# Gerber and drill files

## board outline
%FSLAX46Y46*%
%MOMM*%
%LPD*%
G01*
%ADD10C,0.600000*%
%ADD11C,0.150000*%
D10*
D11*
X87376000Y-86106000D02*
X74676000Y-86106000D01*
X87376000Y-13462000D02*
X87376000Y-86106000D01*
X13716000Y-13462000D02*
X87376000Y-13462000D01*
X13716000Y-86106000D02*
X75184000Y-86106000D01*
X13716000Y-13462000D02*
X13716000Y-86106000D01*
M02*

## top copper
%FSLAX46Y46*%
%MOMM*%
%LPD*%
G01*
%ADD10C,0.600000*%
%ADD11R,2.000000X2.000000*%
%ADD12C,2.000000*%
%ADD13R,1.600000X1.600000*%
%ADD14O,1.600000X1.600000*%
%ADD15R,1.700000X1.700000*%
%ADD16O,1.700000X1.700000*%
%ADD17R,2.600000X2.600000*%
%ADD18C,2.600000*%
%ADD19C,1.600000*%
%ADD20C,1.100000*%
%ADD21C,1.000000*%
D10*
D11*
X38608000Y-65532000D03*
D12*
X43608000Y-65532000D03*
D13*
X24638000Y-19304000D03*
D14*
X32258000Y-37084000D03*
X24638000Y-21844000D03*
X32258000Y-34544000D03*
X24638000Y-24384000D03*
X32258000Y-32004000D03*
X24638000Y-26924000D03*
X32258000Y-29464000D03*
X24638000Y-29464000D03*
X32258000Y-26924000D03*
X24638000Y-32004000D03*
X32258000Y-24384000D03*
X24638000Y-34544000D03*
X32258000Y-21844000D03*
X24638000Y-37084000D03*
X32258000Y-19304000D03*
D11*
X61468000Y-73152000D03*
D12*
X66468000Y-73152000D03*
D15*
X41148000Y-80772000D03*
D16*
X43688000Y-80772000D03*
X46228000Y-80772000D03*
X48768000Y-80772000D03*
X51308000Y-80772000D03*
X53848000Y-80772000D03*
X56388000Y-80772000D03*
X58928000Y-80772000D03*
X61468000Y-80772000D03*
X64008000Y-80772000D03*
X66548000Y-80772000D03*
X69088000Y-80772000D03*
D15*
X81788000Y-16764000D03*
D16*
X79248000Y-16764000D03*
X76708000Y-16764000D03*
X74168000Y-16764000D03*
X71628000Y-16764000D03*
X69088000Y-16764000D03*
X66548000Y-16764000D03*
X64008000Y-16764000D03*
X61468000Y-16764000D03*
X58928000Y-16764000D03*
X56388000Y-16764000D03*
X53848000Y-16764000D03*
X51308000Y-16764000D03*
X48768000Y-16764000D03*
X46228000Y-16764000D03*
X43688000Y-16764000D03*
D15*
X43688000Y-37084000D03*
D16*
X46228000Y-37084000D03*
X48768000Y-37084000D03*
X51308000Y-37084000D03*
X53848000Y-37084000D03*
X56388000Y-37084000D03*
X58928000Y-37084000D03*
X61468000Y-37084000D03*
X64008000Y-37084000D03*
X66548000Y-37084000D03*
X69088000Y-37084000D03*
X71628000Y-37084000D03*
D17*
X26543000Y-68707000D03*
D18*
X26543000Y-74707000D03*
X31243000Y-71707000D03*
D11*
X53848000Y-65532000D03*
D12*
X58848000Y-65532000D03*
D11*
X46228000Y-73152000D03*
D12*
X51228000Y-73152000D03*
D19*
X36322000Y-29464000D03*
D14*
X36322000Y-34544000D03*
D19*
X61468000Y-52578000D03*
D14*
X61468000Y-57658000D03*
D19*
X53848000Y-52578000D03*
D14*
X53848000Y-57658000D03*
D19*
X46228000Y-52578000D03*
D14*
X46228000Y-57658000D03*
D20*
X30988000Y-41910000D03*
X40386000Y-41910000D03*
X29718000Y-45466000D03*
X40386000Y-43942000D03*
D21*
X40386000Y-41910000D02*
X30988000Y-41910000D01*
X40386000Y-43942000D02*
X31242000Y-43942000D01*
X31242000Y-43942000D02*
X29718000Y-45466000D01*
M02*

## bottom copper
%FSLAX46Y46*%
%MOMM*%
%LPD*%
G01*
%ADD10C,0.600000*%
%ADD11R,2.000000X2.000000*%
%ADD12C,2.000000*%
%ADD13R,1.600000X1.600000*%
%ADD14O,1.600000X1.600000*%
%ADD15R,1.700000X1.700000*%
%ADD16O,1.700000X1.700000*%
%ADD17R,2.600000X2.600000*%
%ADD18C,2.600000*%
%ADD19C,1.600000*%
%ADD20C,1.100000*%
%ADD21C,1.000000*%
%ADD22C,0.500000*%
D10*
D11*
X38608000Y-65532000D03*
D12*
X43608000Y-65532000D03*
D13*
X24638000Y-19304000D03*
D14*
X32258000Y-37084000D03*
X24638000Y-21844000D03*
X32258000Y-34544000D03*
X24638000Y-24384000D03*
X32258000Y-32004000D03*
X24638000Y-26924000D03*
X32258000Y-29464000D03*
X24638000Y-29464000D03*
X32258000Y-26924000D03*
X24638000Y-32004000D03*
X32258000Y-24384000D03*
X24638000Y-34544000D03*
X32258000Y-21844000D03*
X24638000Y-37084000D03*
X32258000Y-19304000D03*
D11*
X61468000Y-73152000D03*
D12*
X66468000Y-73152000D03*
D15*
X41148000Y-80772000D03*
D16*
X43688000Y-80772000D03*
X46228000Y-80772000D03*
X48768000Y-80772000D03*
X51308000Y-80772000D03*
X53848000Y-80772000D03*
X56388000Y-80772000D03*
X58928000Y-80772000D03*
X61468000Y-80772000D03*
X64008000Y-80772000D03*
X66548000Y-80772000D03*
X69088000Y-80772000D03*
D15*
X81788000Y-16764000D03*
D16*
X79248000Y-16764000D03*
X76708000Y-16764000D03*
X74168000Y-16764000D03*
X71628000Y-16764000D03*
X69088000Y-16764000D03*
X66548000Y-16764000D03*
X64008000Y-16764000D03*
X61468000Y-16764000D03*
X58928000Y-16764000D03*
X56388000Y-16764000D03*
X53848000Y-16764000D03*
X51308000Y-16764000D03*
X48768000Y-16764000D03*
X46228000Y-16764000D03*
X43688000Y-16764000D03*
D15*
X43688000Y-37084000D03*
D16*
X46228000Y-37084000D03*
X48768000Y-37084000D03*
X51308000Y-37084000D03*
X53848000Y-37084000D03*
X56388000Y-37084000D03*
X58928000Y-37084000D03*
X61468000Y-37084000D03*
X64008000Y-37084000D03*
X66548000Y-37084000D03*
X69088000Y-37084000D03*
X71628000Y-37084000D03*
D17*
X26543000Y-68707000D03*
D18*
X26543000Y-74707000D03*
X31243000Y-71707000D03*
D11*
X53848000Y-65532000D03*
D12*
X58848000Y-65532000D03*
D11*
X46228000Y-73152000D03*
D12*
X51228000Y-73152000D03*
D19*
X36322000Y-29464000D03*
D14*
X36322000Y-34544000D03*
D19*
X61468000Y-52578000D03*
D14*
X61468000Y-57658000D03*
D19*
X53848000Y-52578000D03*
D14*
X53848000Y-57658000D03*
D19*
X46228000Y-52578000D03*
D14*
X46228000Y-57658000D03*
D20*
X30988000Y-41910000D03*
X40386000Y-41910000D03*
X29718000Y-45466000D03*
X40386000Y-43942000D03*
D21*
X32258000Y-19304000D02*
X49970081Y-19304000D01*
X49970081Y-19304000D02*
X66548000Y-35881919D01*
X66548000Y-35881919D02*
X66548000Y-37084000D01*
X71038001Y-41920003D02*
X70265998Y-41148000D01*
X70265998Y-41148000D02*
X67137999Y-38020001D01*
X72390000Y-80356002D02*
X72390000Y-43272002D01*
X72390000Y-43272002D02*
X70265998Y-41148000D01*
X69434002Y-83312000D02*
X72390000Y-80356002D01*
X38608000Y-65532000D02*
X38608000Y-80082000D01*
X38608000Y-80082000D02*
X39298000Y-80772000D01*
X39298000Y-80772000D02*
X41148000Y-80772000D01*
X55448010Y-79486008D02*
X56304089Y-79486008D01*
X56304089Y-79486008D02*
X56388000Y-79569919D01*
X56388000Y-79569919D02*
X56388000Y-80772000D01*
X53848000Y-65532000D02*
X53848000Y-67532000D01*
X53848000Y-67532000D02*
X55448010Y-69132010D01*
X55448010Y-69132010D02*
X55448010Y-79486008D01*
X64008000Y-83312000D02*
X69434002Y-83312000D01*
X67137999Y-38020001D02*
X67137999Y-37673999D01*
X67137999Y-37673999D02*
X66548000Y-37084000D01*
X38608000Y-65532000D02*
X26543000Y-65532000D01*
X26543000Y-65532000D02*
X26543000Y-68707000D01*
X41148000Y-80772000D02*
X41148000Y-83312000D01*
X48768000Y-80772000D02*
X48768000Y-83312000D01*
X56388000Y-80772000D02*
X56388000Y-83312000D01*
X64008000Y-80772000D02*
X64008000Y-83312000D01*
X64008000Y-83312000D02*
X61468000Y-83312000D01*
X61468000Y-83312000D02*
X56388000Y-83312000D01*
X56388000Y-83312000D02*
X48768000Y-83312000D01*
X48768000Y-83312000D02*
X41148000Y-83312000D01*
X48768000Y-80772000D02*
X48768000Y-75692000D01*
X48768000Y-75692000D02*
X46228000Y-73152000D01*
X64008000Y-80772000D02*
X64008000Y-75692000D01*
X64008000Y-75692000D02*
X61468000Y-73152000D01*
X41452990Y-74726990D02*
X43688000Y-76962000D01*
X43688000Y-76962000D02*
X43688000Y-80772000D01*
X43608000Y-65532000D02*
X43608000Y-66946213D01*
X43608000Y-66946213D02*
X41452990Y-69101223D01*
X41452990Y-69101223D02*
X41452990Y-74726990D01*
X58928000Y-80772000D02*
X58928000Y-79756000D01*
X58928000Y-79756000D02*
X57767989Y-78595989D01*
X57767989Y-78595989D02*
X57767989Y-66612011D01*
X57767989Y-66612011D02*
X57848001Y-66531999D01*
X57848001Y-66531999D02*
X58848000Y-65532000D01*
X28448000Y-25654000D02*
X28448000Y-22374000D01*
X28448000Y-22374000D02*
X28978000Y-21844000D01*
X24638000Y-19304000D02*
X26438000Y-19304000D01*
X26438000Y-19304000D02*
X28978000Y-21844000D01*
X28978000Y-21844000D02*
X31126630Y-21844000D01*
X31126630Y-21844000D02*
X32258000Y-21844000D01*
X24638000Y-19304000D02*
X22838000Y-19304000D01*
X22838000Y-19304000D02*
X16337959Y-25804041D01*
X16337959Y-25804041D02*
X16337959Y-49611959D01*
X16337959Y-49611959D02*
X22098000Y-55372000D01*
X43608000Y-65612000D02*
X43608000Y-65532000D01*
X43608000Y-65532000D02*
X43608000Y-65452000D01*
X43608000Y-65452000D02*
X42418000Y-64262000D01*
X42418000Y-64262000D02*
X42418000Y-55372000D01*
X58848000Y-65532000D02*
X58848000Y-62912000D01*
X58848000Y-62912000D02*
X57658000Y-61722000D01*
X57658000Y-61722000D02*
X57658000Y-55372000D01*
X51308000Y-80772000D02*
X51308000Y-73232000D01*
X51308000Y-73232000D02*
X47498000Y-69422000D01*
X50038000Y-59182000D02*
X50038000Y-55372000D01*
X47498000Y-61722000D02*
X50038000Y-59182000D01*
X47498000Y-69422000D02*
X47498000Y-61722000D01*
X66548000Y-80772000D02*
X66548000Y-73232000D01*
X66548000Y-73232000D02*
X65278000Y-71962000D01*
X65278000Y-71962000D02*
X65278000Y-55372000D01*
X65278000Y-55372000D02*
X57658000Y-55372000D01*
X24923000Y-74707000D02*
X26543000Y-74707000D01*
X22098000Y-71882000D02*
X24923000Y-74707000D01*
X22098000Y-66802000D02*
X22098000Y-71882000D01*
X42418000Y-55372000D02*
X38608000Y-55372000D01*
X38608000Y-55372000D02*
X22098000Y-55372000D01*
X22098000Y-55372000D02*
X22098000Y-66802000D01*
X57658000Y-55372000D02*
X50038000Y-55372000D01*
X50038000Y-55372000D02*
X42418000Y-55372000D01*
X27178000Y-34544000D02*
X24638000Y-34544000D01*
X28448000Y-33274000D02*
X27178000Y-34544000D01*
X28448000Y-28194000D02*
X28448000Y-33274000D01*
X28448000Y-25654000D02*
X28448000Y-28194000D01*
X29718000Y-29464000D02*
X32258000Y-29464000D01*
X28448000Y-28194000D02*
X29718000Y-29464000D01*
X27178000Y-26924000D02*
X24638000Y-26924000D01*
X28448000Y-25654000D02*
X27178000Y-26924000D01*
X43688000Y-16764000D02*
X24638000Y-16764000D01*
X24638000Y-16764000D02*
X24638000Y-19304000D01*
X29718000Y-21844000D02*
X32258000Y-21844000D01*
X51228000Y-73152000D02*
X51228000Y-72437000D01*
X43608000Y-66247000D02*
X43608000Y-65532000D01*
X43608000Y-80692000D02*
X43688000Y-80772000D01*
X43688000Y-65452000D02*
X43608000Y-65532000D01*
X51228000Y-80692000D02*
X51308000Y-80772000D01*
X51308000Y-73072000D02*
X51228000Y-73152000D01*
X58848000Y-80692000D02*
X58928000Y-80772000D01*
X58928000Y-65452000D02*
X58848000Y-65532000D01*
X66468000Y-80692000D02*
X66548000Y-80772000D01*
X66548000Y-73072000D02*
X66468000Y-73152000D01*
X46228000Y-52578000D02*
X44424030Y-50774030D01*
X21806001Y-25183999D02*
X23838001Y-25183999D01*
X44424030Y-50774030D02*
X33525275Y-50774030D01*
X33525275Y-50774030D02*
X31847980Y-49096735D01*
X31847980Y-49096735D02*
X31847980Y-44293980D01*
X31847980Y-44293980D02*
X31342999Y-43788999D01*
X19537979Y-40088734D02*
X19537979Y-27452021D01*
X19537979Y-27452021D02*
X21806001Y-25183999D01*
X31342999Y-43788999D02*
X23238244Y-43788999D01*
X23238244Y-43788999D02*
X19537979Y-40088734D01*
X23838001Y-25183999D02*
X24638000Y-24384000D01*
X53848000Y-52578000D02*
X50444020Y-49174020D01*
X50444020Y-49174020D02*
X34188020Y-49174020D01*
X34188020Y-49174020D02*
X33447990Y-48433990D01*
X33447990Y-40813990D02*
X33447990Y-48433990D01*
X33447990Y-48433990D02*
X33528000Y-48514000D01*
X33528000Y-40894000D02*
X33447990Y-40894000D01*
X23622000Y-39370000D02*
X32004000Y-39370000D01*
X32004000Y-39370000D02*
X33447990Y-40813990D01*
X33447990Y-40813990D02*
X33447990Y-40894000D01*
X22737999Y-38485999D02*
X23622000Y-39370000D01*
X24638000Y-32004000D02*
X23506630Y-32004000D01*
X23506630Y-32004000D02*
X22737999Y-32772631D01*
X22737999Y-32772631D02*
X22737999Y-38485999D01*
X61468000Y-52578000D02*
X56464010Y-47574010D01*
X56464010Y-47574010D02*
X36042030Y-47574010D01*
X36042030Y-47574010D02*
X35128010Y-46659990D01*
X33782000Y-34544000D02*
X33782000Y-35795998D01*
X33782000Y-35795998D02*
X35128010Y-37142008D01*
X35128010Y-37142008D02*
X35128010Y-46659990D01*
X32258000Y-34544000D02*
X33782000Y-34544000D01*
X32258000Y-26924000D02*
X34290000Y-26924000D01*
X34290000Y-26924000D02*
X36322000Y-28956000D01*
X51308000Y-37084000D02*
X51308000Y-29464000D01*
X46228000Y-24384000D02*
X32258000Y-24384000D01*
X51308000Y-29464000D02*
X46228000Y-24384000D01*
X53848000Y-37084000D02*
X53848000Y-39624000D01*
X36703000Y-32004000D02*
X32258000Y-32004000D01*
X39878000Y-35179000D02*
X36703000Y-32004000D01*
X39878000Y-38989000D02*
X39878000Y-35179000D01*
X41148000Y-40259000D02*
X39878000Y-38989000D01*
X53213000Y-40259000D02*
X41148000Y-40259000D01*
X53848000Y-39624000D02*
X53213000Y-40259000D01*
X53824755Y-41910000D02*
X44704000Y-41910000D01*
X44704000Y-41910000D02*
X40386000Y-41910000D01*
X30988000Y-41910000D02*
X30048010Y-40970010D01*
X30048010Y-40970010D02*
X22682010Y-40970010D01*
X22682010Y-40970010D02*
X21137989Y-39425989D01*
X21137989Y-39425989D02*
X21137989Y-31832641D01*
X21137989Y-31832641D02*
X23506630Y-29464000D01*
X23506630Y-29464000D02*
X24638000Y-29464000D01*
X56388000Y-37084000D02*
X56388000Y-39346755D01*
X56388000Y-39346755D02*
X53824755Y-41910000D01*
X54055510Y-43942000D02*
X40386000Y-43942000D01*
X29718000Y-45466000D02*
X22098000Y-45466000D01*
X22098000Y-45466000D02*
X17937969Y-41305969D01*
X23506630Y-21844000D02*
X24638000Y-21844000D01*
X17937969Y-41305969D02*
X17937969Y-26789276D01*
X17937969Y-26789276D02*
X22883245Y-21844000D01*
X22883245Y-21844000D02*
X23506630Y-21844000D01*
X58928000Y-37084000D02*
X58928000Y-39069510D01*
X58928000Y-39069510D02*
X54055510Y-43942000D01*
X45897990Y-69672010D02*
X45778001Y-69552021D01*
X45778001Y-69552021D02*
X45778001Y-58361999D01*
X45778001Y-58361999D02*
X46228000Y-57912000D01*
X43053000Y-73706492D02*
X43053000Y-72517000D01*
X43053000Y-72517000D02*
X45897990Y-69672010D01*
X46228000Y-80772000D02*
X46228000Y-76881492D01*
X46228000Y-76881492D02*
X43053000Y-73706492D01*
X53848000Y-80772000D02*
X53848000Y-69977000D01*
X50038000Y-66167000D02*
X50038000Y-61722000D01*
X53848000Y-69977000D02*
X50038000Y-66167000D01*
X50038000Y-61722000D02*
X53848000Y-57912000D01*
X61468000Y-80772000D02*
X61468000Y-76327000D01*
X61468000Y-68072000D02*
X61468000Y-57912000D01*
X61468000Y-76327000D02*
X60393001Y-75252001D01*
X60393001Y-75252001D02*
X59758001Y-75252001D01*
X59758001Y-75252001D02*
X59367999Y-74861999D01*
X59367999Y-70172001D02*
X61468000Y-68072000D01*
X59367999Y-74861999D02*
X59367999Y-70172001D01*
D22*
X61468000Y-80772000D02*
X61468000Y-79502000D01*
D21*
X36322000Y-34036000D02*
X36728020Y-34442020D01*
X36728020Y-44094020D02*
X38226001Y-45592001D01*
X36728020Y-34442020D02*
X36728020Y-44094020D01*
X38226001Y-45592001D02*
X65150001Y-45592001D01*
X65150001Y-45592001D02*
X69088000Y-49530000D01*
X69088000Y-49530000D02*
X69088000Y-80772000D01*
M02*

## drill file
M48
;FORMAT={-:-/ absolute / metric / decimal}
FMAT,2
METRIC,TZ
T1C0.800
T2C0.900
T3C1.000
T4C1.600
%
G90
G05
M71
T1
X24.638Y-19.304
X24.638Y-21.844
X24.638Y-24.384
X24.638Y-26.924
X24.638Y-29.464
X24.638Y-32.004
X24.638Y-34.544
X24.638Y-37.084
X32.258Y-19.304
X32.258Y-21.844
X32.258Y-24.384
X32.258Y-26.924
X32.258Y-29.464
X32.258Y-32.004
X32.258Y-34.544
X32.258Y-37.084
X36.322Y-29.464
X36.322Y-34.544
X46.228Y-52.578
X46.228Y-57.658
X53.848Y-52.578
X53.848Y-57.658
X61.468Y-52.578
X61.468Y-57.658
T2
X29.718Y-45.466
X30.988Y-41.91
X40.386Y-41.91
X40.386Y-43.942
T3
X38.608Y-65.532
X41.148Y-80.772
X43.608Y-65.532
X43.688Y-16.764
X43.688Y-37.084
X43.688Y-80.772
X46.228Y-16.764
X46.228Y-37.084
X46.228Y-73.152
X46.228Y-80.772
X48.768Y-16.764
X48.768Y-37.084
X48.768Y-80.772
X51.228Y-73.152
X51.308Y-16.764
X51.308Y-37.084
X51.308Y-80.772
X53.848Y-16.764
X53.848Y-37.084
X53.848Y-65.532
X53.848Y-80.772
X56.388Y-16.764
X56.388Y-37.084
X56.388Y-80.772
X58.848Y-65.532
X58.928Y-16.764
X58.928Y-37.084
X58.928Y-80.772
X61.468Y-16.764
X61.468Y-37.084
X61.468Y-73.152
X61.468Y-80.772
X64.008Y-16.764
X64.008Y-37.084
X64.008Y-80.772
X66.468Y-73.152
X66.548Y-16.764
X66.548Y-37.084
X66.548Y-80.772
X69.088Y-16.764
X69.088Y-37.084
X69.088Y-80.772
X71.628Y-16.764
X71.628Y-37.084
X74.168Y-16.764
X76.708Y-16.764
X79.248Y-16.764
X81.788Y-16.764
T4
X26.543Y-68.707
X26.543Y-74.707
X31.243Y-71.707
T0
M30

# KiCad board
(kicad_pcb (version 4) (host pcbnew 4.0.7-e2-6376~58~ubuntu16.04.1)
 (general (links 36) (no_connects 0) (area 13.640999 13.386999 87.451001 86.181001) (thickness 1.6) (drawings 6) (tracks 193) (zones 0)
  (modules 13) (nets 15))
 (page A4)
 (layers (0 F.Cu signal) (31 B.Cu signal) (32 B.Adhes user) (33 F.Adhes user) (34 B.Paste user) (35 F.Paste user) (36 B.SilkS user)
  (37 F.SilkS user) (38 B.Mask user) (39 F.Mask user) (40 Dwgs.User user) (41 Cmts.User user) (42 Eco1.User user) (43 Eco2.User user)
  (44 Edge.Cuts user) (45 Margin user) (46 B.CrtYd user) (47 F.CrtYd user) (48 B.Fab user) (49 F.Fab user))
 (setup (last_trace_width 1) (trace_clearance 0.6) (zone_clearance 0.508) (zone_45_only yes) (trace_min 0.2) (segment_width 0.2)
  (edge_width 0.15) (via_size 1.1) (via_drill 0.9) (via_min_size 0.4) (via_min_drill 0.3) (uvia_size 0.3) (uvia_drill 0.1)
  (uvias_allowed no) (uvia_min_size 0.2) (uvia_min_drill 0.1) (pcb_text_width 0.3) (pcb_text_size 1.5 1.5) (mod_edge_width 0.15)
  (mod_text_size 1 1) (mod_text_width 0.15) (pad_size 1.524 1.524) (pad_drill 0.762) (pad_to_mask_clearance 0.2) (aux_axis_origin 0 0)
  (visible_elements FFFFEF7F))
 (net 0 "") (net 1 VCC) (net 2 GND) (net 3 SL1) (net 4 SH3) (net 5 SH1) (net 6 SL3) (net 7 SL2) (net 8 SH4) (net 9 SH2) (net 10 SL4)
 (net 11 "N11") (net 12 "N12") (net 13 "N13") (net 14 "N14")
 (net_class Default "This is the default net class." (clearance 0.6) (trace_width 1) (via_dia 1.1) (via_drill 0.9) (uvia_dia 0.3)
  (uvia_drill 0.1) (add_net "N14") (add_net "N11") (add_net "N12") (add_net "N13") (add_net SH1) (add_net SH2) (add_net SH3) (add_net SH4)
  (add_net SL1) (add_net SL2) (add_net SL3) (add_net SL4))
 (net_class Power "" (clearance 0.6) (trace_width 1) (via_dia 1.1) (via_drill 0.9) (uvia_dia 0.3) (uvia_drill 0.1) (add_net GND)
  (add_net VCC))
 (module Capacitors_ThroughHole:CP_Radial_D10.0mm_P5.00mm (layer F.Cu) (at 38.608 65.532)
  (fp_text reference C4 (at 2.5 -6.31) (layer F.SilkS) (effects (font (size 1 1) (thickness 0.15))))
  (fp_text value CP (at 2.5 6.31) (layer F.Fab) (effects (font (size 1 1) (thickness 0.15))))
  (pad 1 thru_hole rect (at 0 0) (size 2 2) (drill 1) (layers *.Cu *.Mask) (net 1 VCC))
  (pad 2 thru_hole circle (at 5 0) (size 2 2) (drill 1) (layers *.Cu *.Mask) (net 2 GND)))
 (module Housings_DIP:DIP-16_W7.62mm (layer F.Cu) (at 24.638 19.304)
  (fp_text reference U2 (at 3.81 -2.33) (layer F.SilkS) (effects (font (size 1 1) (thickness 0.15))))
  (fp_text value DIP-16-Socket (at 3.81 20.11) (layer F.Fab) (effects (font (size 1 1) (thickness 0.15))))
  (pad 1 thru_hole rect (at 0 0) (size 1.6 1.6) (drill 0.8) (layers *.Cu *.Mask) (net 2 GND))
  (pad 9 thru_hole oval (at 7.62 17.78) (size 1.6 1.6) (drill 0.8) (layers *.Cu *.Mask))
  (pad 2 thru_hole oval (at 0 2.54) (size 1.6 1.6) (drill 0.8) (layers *.Cu *.Mask) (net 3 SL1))
  (pad 10 thru_hole oval (at 7.62 15.24) (size 1.6 1.6) (drill 0.8) (layers *.Cu *.Mask) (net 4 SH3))
  (pad 3 thru_hole oval (at 0 5.08) (size 1.6 1.6) (drill 0.8) (layers *.Cu *.Mask) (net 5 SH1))
  (pad 11 thru_hole oval (at 7.62 12.7) (size 1.6 1.6) (drill 0.8) (layers *.Cu *.Mask) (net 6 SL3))
  (pad 4 thru_hole oval (at 0 7.62) (size 1.6 1.6) (drill 0.8) (layers *.Cu *.Mask) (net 2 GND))
  (pad 12 thru_hole oval (at 7.62 10.16) (size 1.6 1.6) (drill 0.8) (layers *.Cu *.Mask) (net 2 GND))
  (pad 5 thru_hole oval (at 0 10.16) (size 1.6 1.6) (drill 0.8) (layers *.Cu *.Mask) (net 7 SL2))
  (pad 13 thru_hole oval (at 7.62 7.62) (size 1.6 1.6) (drill 0.8) (layers *.Cu *.Mask) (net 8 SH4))
  (pad 6 thru_hole oval (at 0 12.7) (size 1.6 1.6) (drill 0.8) (layers *.Cu *.Mask) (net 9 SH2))
  (pad 14 thru_hole oval (at 7.62 5.08) (size 1.6 1.6) (drill 0.8) (layers *.Cu *.Mask) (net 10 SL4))
  (pad 7 thru_hole oval (at 0 15.24) (size 1.6 1.6) (drill 0.8) (layers *.Cu *.Mask) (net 2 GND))
  (pad 15 thru_hole oval (at 7.62 2.54) (size 1.6 1.6) (drill 0.8) (layers *.Cu *.Mask) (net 2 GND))
  (pad 8 thru_hole oval (at 0 17.78) (size 1.6 1.6) (drill 0.8) (layers *.Cu *.Mask))
  (pad 16 thru_hole oval (at 7.62 0) (size 1.6 1.6) (drill 0.8) (layers *.Cu *.Mask) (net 1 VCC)))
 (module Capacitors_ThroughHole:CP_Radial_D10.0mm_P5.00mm (layer F.Cu) (at 61.468 73.152)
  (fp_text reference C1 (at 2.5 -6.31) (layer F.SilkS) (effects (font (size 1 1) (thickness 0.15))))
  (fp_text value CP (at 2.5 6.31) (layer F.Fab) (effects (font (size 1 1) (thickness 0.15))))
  (pad 1 thru_hole rect (at 0 0) (size 2 2) (drill 1) (layers *.Cu *.Mask) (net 1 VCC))
  (pad 2 thru_hole circle (at 5 0) (size 2 2) (drill 1) (layers *.Cu *.Mask) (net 2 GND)))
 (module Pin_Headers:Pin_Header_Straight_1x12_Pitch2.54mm (layer F.Cu) (at 41.148 80.772 90)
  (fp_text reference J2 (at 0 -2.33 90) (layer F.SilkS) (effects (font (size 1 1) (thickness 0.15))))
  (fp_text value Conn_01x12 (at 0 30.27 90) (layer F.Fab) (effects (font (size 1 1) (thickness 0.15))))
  (pad 1 thru_hole rect (at 0 0 90) (size 1.7 1.7) (drill 1) (layers *.Cu *.Mask) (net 1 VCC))
  (pad 2 thru_hole oval (at 0 2.54 90) (size 1.7 1.7) (drill 1) (layers *.Cu *.Mask) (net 2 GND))
  (pad 3 thru_hole oval (at 0 5.08 90) (size 1.7 1.7) (drill 1) (layers *.Cu *.Mask) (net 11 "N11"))
  (pad 4 thru_hole oval (at 0 7.62 90) (size 1.7 1.7) (drill 1) (layers *.Cu *.Mask) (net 1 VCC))
  (pad 5 thru_hole oval (at 0 10.16 90) (size 1.7 1.7) (drill 1) (layers *.Cu *.Mask) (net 2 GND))
  (pad 6 thru_hole oval (at 0 12.7 90) (size 1.7 1.7) (drill 1) (layers *.Cu *.Mask) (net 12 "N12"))
  (pad 7 thru_hole oval (at 0 15.24 90) (size 1.7 1.7) (drill 1) (layers *.Cu *.Mask) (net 1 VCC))
  (pad 8 thru_hole oval (at 0 17.78 90) (size 1.7 1.7) (drill 1) (layers *.Cu *.Mask) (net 2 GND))
  (pad 9 thru_hole oval (at 0 20.32 90) (size 1.7 1.7) (drill 1) (layers *.Cu *.Mask) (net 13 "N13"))
  (pad 10 thru_hole oval (at 0 22.86 90) (size 1.7 1.7) (drill 1) (layers *.Cu *.Mask) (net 1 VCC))
  (pad 11 thru_hole oval (at 0 25.4 90) (size 1.7 1.7) (drill 1) (layers *.Cu *.Mask) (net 2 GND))
  (pad 12 thru_hole oval (at 0 27.94 90) (size 1.7 1.7) (drill 1) (layers *.Cu *.Mask) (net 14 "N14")))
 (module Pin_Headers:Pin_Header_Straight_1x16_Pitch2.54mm (layer F.Cu) (at 81.788 16.764 270)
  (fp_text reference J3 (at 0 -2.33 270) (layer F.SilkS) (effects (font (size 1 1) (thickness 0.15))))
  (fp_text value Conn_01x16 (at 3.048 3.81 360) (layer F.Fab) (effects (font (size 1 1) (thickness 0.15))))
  (pad 1 thru_hole rect (at 0 0 270) (size 1.7 1.7) (drill 1) (layers *.Cu *.Mask))
  (pad 2 thru_hole oval (at 0 2.54 270) (size 1.7 1.7) (drill 1) (layers *.Cu *.Mask))
  (pad 3 thru_hole oval (at 0 5.08 270) (size 1.7 1.7) (drill 1) (layers *.Cu *.Mask))
  (pad 4 thru_hole oval (at 0 7.62 270) (size 1.7 1.7) (drill 1) (layers *.Cu *.Mask))
  (pad 5 thru_hole oval (at 0 10.16 270) (size 1.7 1.7) (drill 1) (layers *.Cu *.Mask))
  (pad 6 thru_hole oval (at 0 12.7 270) (size 1.7 1.7) (drill 1) (layers *.Cu *.Mask))
  (pad 7 thru_hole oval (at 0 15.24 270) (size 1.7 1.7) (drill 1) (layers *.Cu *.Mask))
  (pad 8 thru_hole oval (at 0 17.78 270) (size 1.7 1.7) (drill 1) (layers *.Cu *.Mask))
  (pad 9 thru_hole oval (at 0 20.32 270) (size 1.7 1.7) (drill 1) (layers *.Cu *.Mask))
  (pad 10 thru_hole oval (at 0 22.86 270) (size 1.7 1.7) (drill 1) (layers *.Cu *.Mask))
  (pad 11 thru_hole oval (at 0 25.4 270) (size 1.7 1.7) (drill 1) (layers *.Cu *.Mask))
  (pad 12 thru_hole oval (at 0 27.94 270) (size 1.7 1.7) (drill 1) (layers *.Cu *.Mask))
  (pad 13 thru_hole oval (at 0 30.48 270) (size 1.7 1.7) (drill 1) (layers *.Cu *.Mask))
  (pad 14 thru_hole oval (at 0 33.02 270) (size 1.7 1.7) (drill 1) (layers *.Cu *.Mask))
  (pad 15 thru_hole oval (at 0 35.56 270) (size 1.7 1.7) (drill 1) (layers *.Cu *.Mask))
  (pad 16 thru_hole oval (at 0 38.1 270) (size 1.7 1.7) (drill 1) (layers *.Cu *.Mask) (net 2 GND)))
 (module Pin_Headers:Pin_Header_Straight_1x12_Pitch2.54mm (layer F.Cu) (at 43.688 37.084 90)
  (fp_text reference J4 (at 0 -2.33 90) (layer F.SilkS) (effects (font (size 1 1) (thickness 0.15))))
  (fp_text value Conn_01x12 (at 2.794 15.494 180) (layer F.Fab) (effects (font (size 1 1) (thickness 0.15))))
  (pad 1 thru_hole rect (at 0 0 90) (size 1.7 1.7) (drill 1) (layers *.Cu *.Mask))
  (pad 2 thru_hole oval (at 0 2.54 90) (size 1.7 1.7) (drill 1) (layers *.Cu *.Mask))
  (pad 3 thru_hole oval (at 0 5.08 90) (size 1.7 1.7) (drill 1) (layers *.Cu *.Mask))
  (pad 4 thru_hole oval (at 0 7.62 90) (size 1.7 1.7) (drill 1) (layers *.Cu *.Mask) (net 10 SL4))
  (pad 5 thru_hole oval (at 0 10.16 90) (size 1.7 1.7) (drill 1) (layers *.Cu *.Mask) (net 6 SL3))
  (pad 6 thru_hole oval (at 0 12.7 90) (size 1.7 1.7) (drill 1) (layers *.Cu *.Mask) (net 7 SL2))
  (pad 7 thru_hole oval (at 0 15.24 90) (size 1.7 1.7) (drill 1) (layers *.Cu *.Mask) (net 3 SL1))
  (pad 8 thru_hole oval (at 0 17.78 90) (size 1.7 1.7) (drill 1) (layers *.Cu *.Mask))
  (pad 9 thru_hole oval (at 0 20.32 90) (size 1.7 1.7) (drill 1) (layers *.Cu *.Mask))
  (pad 10 thru_hole oval (at 0 22.86 90) (size 1.7 1.7) (drill 1) (layers *.Cu *.Mask) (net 1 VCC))
  (pad 11 thru_hole oval (at 0 25.4 90) (size 1.7 1.7) (drill 1) (layers *.Cu *.Mask))
  (pad 12 thru_hole oval (at 0 27.94 90) (size 1.7 1.7) (drill 1) (layers *.Cu *.Mask)))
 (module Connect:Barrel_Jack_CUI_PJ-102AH (layer F.Cu) (at 26.543 68.707)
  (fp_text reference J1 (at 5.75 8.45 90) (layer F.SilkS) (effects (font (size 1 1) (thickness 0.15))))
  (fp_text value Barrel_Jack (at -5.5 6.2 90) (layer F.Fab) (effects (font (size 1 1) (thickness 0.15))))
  (pad 1 thru_hole rect (at 0 0) (size 2.6 2.6) (drill 1.6) (layers *.Cu *.Mask) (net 1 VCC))
  (pad 2 thru_hole circle (at 0 6) (size 2.6 2.6) (drill 1.6) (layers *.Cu *.Mask) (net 2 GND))
  (pad 3 thru_hole circle (at 4.7 3) (size 2.6 2.6) (drill 1.6) (layers *.Cu *.Mask)))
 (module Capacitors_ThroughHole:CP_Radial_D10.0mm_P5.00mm (layer F.Cu) (at 53.848 65.532)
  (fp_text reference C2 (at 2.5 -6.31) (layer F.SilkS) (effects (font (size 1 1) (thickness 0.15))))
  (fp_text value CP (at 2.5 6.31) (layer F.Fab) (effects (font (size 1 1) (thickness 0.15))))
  (pad 1 thru_hole rect (at 0 0) (size 2 2) (drill 1) (layers *.Cu *.Mask) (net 1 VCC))
  (pad 2 thru_hole circle (at 5 0) (size 2 2) (drill 1) (layers *.Cu *.Mask) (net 2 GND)))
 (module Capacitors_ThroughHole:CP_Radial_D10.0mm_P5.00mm (layer F.Cu) (at 46.228 73.152)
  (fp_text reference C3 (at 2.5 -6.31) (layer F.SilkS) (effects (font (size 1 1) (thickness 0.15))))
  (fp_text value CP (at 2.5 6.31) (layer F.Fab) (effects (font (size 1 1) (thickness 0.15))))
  (pad 1 thru_hole rect (at 0 0) (size 2 2) (drill 1) (layers *.Cu *.Mask) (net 1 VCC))
  (pad 2 thru_hole circle (at 5 0) (size 2 2) (drill 1) (layers *.Cu *.Mask) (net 2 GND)))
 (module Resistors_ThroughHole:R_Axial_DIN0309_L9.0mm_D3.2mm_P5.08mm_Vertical (layer F.Cu) (at 36.322 29.464 270)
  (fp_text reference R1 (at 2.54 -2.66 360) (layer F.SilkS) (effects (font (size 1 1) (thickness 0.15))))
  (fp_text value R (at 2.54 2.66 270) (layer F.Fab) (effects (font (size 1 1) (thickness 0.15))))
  (pad 1 thru_hole circle (at 0 0 270) (size 1.6 1.6) (drill 0.8) (layers *.Cu *.Mask) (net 8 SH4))
  (pad 2 thru_hole oval (at 5.08 0 270) (size 1.6 1.6) (drill 0.8) (layers *.Cu *.Mask) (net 14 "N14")))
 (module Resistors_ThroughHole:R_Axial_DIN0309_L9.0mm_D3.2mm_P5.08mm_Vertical (layer F.Cu) (at 61.468 52.578 270)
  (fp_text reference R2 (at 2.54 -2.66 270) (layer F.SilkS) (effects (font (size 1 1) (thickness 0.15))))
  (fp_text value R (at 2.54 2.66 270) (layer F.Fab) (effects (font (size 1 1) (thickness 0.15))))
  (pad 1 thru_hole circle (at 0 0 270) (size 1.6 1.6) (drill 0.8) (layers *.Cu *.Mask) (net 4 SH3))
  (pad 2 thru_hole oval (at 5.08 0 270) (size 1.6 1.6) (drill 0.8) (layers *.Cu *.Mask) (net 13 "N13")))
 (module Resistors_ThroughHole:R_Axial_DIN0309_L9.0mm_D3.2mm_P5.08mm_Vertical (layer F.Cu) (at 53.848 52.578 270)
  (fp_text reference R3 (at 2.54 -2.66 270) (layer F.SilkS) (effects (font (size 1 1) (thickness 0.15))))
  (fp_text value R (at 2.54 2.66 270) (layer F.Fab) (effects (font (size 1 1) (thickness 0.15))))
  (pad 1 thru_hole circle (at 0 0 270) (size 1.6 1.6) (drill 0.8) (layers *.Cu *.Mask) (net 9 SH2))
  (pad 2 thru_hole oval (at 5.08 0 270) (size 1.6 1.6) (drill 0.8) (layers *.Cu *.Mask) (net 12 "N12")))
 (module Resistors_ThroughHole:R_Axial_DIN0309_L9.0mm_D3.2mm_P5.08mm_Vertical (layer F.Cu) (at 46.228 52.578 270)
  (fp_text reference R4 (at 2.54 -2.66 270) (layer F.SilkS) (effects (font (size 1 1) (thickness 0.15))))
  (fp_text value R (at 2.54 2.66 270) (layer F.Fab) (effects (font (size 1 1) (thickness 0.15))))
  (pad 1 thru_hole circle (at 0 0 270) (size 1.6 1.6) (drill 0.8) (layers *.Cu *.Mask) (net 5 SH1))
  (pad 2 thru_hole oval (at 5.08 0 270) (size 1.6 1.6) (drill 0.8) (layers *.Cu *.Mask) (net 11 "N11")))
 (gr_line (start 87.376 86.106) (end 74.676 86.106) (layer Edge.Cuts) (width 0.15))
 (gr_line (start 87.376 13.462) (end 87.376 86.106) (layer Edge.Cuts) (width 0.15))
 (gr_line (start 13.716 13.462) (end 87.376 13.462) (layer Edge.Cuts) (width 0.15))
 (gr_line (start 13.716 86.106) (end 75.184 86.106) (layer Edge.Cuts) (width 0.15))
 (gr_line (start 13.716 13.462) (end 13.716 86.106) (layer Edge.Cuts) (width 0.15))
 (segment (start 32.258 19.304) (end 49.970081 19.304) (width 1) (layer B.Cu) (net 1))
 (segment (start 49.970081 19.304) (end 66.548 35.881919) (width 1) (layer B.Cu) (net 1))
 (segment (start 66.548 35.881919) (end 66.548 37.084) (width 1) (layer B.Cu) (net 1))
 (segment (start 71.038001 41.920003) (end 70.265998 41.148) (width 1) (layer B.Cu) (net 1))
 (segment (start 70.265998 41.148) (end 67.137999 38.020001) (width 1) (layer B.Cu) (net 1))
 (segment (start 72.39 80.356002) (end 72.39 43.272002) (width 1) (layer B.Cu) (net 1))
 (segment (start 72.39 43.272002) (end 70.265998 41.148) (width 1) (layer B.Cu) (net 1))
 (segment (start 69.434002 83.312) (end 72.39 80.356002) (width 1) (layer B.Cu) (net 1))
 (segment (start 38.608 65.532) (end 38.608 80.082) (width 1) (layer B.Cu) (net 1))
 (segment (start 38.608 80.082) (end 39.298 80.772) (width 1) (layer B.Cu) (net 1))
 (segment (start 39.298 80.772) (end 41.148 80.772) (width 1) (layer B.Cu) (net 1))
 (segment (start 55.44801 79.486008) (end 56.304089 79.486008) (width 1) (layer B.Cu) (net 1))
 (segment (start 56.304089 79.486008) (end 56.388 79.569919) (width 1) (layer B.Cu) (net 1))
 (segment (start 56.388 79.569919) (end 56.388 80.772) (width 1) (layer B.Cu) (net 1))
 (segment (start 53.848 65.532) (end 53.848 67.532) (width 1) (layer B.Cu) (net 1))
 (segment (start 53.848 67.532) (end 55.44801 69.13201) (width 1) (layer B.Cu) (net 1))
 (segment (start 55.44801 69.13201) (end 55.44801 79.486008) (width 1) (layer B.Cu) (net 1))
 (segment (start 64.008 83.312) (end 69.434002 83.312) (width 1) (layer B.Cu) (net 1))
 (segment (start 67.137999 38.020001) (end 67.137999 37.673999) (width 1) (layer B.Cu) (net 1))
 (segment (start 67.137999 37.673999) (end 66.548 37.084) (width 1) (layer B.Cu) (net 1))
 (segment (start 38.608 65.532) (end 26.543 65.532) (width 1) (layer B.Cu) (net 1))
 (segment (start 26.543 65.532) (end 26.543 68.707) (width 1) (layer B.Cu) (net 1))
 (segment (start 41.148 80.772) (end 41.148 83.312) (width 1) (layer B.Cu) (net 1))
 (segment (start 48.768 80.772) (end 48.768 83.312) (width 1) (layer B.Cu) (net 1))
 (segment (start 56.388 80.772) (end 56.388 83.312) (width 1) (layer B.Cu) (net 1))
 (segment (start 64.008 80.772) (end 64.008 83.312) (width 1) (layer B.Cu) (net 1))
 (segment (start 64.008 83.312) (end 61.468 83.312) (width 1) (layer B.Cu) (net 1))
 (segment (start 61.468 83.312) (end 56.388 83.312) (width 1) (layer B.Cu) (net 1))
 (segment (start 56.388 83.312) (end 48.768 83.312) (width 1) (layer B.Cu) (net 1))
 (segment (start 48.768 83.312) (end 41.148 83.312) (width 1) (layer B.Cu) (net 1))
 (segment (start 48.768 80.772) (end 48.768 75.692) (width 1) (layer B.Cu) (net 1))
 (segment (start 48.768 75.692) (end 46.228 73.152) (width 1) (layer B.Cu) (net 1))
 (segment (start 64.008 80.772) (end 64.008 75.692) (width 1) (layer B.Cu) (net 1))
 (segment (start 64.008 75.692) (end 61.468 73.152) (width 1) (layer B.Cu) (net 1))
 (segment (start 41.45299 74.72699) (end 43.688 76.962) (width 1) (layer B.Cu) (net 2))
 (segment (start 43.688 76.962) (end 43.688 80.772) (width 1) (layer B.Cu) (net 2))
 (segment (start 43.608 65.532) (end 43.608 66.946213) (width 1) (layer B.Cu) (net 2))
 (segment (start 43.608 66.946213) (end 41.45299 69.101223) (width 1) (layer B.Cu) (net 2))
 (segment (start 41.45299 69.101223) (end 41.45299 74.72699) (width 1) (layer B.Cu) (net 2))
 (segment (start 58.928 80.772) (end 58.928 79.756) (width 1) (layer B.Cu) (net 2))
 (segment (start 58.928 79.756) (end 57.767989 78.595989) (width 1) (layer B.Cu) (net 2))
 (segment (start 57.767989 78.595989) (end 57.767989 66.612011) (width 1) (layer B.Cu) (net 2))
 (segment (start 57.767989 66.612011) (end 57.848001 66.531999) (width 1) (layer B.Cu) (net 2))
 (segment (start 57.848001 66.531999) (end 58.848 65.532) (width 1) (layer B.Cu) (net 2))
 (segment (start 28.448 25.654) (end 28.448 22.374) (width 1) (layer B.Cu) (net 2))
 (segment (start 28.448 22.374) (end 28.978 21.844) (width 1) (layer B.Cu) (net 2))
 (segment (start 24.638 19.304) (end 26.438 19.304) (width 1) (layer B.Cu) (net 2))
 (segment (start 26.438 19.304) (end 28.978 21.844) (width 1) (layer B.Cu) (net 2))
 (segment (start 28.978 21.844) (end 31.12663 21.844) (width 1) (layer B.Cu) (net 2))
 (segment (start 31.12663 21.844) (end 32.258 21.844) (width 1) (layer B.Cu) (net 2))
 (segment (start 24.638 19.304) (end 22.838 19.304) (width 1) (layer B.Cu) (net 2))
 (segment (start 22.838 19.304) (end 16.337959 25.804041) (width 1) (layer B.Cu) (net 2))
 (segment (start 16.337959 25.804041) (end 16.337959 49.611959) (width 1) (layer B.Cu) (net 2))
 (segment (start 16.337959 49.611959) (end 22.098 55.372) (width 1) (layer B.Cu) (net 2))
 (segment (start 43.608 65.612) (end 43.608 65.532) (width 1) (layer B.Cu) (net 2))
 (segment (start 43.608 65.532) (end 43.608 65.452) (width 1) (layer B.Cu) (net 2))
 (segment (start 43.608 65.452) (end 42.418 64.262) (width 1) (layer B.Cu) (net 2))
 (segment (start 42.418 64.262) (end 42.418 55.372) (width 1) (layer B.Cu) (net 2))
 (segment (start 58.848 65.532) (end 58.848 62.912) (width 1) (layer B.Cu) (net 2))
 (segment (start 58.848 62.912) (end 57.658 61.722) (width 1) (layer B.Cu) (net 2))
 (segment (start 57.658 61.722) (end 57.658 55.372) (width 1) (layer B.Cu) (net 2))
 (segment (start 51.308 80.772) (end 51.308 73.232) (width 1) (layer B.Cu) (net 2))
 (segment (start 51.308 73.232) (end 47.498 69.422) (width 1) (layer B.Cu) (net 2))
 (segment (start 50.038 59.182) (end 50.038 55.372) (width 1) (layer B.Cu) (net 2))
 (segment (start 47.498 61.722) (end 50.038 59.182) (width 1) (layer B.Cu) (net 2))
 (segment (start 47.498 69.422) (end 47.498 61.722) (width 1) (layer B.Cu) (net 2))
 (segment (start 66.548 80.772) (end 66.548 73.232) (width 1) (layer B.Cu) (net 2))
 (segment (start 66.548 73.232) (end 65.278 71.962) (width 1) (layer B.Cu) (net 2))
 (segment (start 65.278 71.962) (end 65.278 55.372) (width 1) (layer B.Cu) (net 2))
 (segment (start 65.278 55.372) (end 57.658 55.372) (width 1) (layer B.Cu) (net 2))
 (segment (start 24.923 74.707) (end 26.543 74.707) (width 1) (layer B.Cu) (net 2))
 (segment (start 22.098 71.882) (end 24.923 74.707) (width 1) (layer B.Cu) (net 2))
 (segment (start 22.098 66.802) (end 22.098 71.882) (width 1) (layer B.Cu) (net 2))
 (segment (start 42.418 55.372) (end 38.608 55.372) (width 1) (layer B.Cu) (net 2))
 (segment (start 38.608 55.372) (end 22.098 55.372) (width 1) (layer B.Cu) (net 2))
 (segment (start 22.098 55.372) (end 22.098 66.802) (width 1) (layer B.Cu) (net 2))
 (segment (start 57.658 55.372) (end 50.038 55.372) (width 1) (layer B.Cu) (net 2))
 (segment (start 50.038 55.372) (end 42.418 55.372) (width 1) (layer B.Cu) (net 2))
 (segment (start 27.178 34.544) (end 24.638 34.544) (width 1) (layer B.Cu) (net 2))
 (segment (start 28.448 33.274) (end 27.178 34.544) (width 1) (layer B.Cu) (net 2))
 (segment (start 28.448 28.194) (end 28.448 33.274) (width 1) (layer B.Cu) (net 2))
 (segment (start 28.448 25.654) (end 28.448 28.194) (width 1) (layer B.Cu) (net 2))
 (segment (start 29.718 29.464) (end 32.258 29.464) (width 1) (layer B.Cu) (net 2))
 (segment (start 28.448 28.194) (end 29.718 29.464) (width 1) (layer B.Cu) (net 2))
 (segment (start 27.178 26.924) (end 24.638 26.924) (width 1) (layer B.Cu) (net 2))
 (segment (start 28.448 25.654) (end 27.178 26.924) (width 1) (layer B.Cu) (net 2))
 (segment (start 43.688 16.764) (end 24.638 16.764) (width 1) (layer B.Cu) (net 2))
 (segment (start 24.638 16.764) (end 24.638 19.304) (width 1) (layer B.Cu) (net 2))
 (segment (start 29.718 21.844) (end 32.258 21.844) (width 1) (layer B.Cu) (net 2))
 (segment (start 51.228 73.152) (end 51.228 72.437) (width 1) (layer B.Cu) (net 2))
 (segment (start 43.608 66.247) (end 43.608 65.532) (width 1) (layer B.Cu) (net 2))
 (segment (start 43.608 80.692) (end 43.688 80.772) (width 1) (layer B.Cu) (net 2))
 (segment (start 43.688 65.452) (end 43.608 65.532) (width 1) (layer B.Cu) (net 2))
 (segment (start 51.228 80.692) (end 51.308 80.772) (width 1) (layer B.Cu) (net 2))
 (segment (start 51.308 73.072) (end 51.228 73.152) (width 1) (layer B.Cu) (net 2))
 (segment (start 58.848 80.692) (end 58.928 80.772) (width 1) (layer B.Cu) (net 2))
 (segment (start 58.928 65.452) (end 58.848 65.532) (width 1) (layer B.Cu) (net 2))
 (segment (start 66.468 80.692) (end 66.548 80.772) (width 1) (layer B.Cu) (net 2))
 (segment (start 66.548 73.072) (end 66.468 73.152) (width 1) (layer B.Cu) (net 2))
 (segment (start 46.228 52.578) (end 44.42403 50.77403) (width 1) (layer B.Cu) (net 5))
 (segment (start 21.806001 25.183999) (end 23.838001 25.183999) (width 1) (layer B.Cu) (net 5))
 (segment (start 44.42403 50.77403) (end 33.525275 50.77403) (width 1) (layer B.Cu) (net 5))
 (segment (start 33.525275 50.77403) (end 31.84798 49.096735) (width 1) (layer B.Cu) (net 5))
 (segment (start 31.84798 49.096735) (end 31.84798 44.29398) (width 1) (layer B.Cu) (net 5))
 (segment (start 31.84798 44.29398) (end 31.342999 43.788999) (width 1) (layer B.Cu) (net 5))
 (segment (start 19.537979 40.088734) (end 19.537979 27.452021) (width 1) (layer B.Cu) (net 5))
 (segment (start 19.537979 27.452021) (end 21.806001 25.183999) (width 1) (layer B.Cu) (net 5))
 (segment (start 31.342999 43.788999) (end 23.238244 43.788999) (width 1) (layer B.Cu) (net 5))
 (segment (start 23.238244 43.788999) (end 19.537979 40.088734) (width 1) (layer B.Cu) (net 5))
 (segment (start 23.838001 25.183999) (end 24.638 24.384) (width 1) (layer B.Cu) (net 5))
 (segment (start 53.848 52.578) (end 50.44402 49.17402) (width 1) (layer B.Cu) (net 9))
 (segment (start 50.44402 49.17402) (end 34.18802 49.17402) (width 1) (layer B.Cu) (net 9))
 (segment (start 34.18802 49.17402) (end 33.44799 48.43399) (width 1) (layer B.Cu) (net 9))
 (segment (start 33.44799 40.81399) (end 33.44799 48.43399) (width 1) (layer B.Cu) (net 9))
 (segment (start 33.44799 48.43399) (end 33.528 48.514) (width 1) (layer B.Cu) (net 9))
 (segment (start 33.528 40.894) (end 33.44799 40.894) (width 1) (layer B.Cu) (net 9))
 (segment (start 23.622 39.37) (end 32.004 39.37) (width 1) (layer B.Cu) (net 9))
 (segment (start 32.004 39.37) (end 33.44799 40.81399) (width 1) (layer B.Cu) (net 9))
 (segment (start 33.44799 40.81399) (end 33.44799 40.894) (width 1) (layer B.Cu) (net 9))
 (segment (start 22.737999 38.485999) (end 23.622 39.37) (width 1) (layer B.Cu) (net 9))
 (segment (start 24.638 32.004) (end 23.50663 32.004) (width 1) (layer B.Cu) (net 9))
 (segment (start 23.50663 32.004) (end 22.737999 32.772631) (width 1) (layer B.Cu) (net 9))
 (segment (start 22.737999 32.772631) (end 22.737999 38.485999) (width 1) (layer B.Cu) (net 9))
 (segment (start 61.468 52.578) (end 56.46401 47.57401) (width 1) (layer B.Cu) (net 4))
 (segment (start 56.46401 47.57401) (end 36.04203 47.57401) (width 1) (layer B.Cu) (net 4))
 (segment (start 36.04203 47.57401) (end 35.12801 46.65999) (width 1) (layer B.Cu) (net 4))
 (segment (start 33.782 34.544) (end 33.782 35.795998) (width 1) (layer B.Cu) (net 4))
 (segment (start 33.782 35.795998) (end 35.12801 37.142008) (width 1) (layer B.Cu) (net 4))
 (segment (start 35.12801 37.142008) (end 35.12801 46.65999) (width 1) (layer B.Cu) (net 4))
 (segment (start 32.258 34.544) (end 33.782 34.544) (width 1) (layer B.Cu) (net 4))
 (segment (start 32.258 26.924) (end 34.29 26.924) (width 1) (layer B.Cu) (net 8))
 (segment (start 34.29 26.924) (end 36.322 28.956) (width 1) (layer B.Cu) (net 8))
 (segment (start 51.308 37.084) (end 51.308 29.464) (width 1) (layer B.Cu) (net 10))
 (segment (start 46.228 24.384) (end 32.258 24.384) (width 1) (layer B.Cu) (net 10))
 (segment (start 51.308 29.464) (end 46.228 24.384) (width 1) (layer B.Cu) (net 10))
 (segment (start 53.848 37.084) (end 53.848 39.624) (width 1) (layer B.Cu) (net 6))
 (segment (start 36.703 32.004) (end 32.258 32.004) (width 1) (layer B.Cu) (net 6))
 (segment (start 39.878 35.179) (end 36.703 32.004) (width 1) (layer B.Cu) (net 6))
 (segment (start 39.878 38.989) (end 39.878 35.179) (width 1) (layer B.Cu) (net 6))
 (segment (start 41.148 40.259) (end 39.878 38.989) (width 1) (layer B.Cu) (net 6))
 (segment (start 53.213 40.259) (end 41.148 40.259) (width 1) (layer B.Cu) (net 6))
 (segment (start 53.848 39.624) (end 53.213 40.259) (width 1) (layer B.Cu) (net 6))
 (segment (start 40.386 41.91) (end 30.988 41.91) (width 1) (layer F.Cu) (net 7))
 (segment (start 53.824755 41.91) (end 44.704 41.91) (width 1) (layer B.Cu) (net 7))
 (segment (start 44.704 41.91) (end 40.386 41.91) (width 1) (layer B.Cu) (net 7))
 (segment (start 30.988 41.91) (end 30.04801 40.97001) (width 1) (layer B.Cu) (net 7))
 (segment (start 30.04801 40.97001) (end 22.68201 40.97001) (width 1) (layer B.Cu) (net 7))
 (segment (start 22.68201 40.97001) (end 21.137989 39.425989) (width 1) (layer B.Cu) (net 7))
 (segment (start 21.137989 39.425989) (end 21.137989 31.832641) (width 1) (layer B.Cu) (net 7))
 (segment (start 21.137989 31.832641) (end 23.50663 29.464) (width 1) (layer B.Cu) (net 7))
 (segment (start 23.50663 29.464) (end 24.638 29.464) (width 1) (layer B.Cu) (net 7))
 (via (at 30.988 41.91) (size 1.1) (drill 0.9) (layers F.Cu B.Cu) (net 7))
 (segment (start 56.388 37.084) (end 56.388 39.346755) (width 1) (layer B.Cu) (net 7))
 (segment (start 56.388 39.346755) (end 53.824755 41.91) (width 1) (layer B.Cu) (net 7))
 (via (at 40.386 41.91) (size 1.1) (drill 0.9) (layers F.Cu B.Cu) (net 7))
 (segment (start 40.386 43.942) (end 31.242 43.942) (width 1) (layer F.Cu) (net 3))
 (segment (start 31.242 43.942) (end 29.718 45.466) (width 1) (layer F.Cu) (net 3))
 (segment (start 54.05551 43.942) (end 40.386 43.942) (width 1) (layer B.Cu) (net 3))
 (segment (start 29.718 45.466) (end 22.098 45.466) (width 1) (layer B.Cu) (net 3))
 (segment (start 22.098 45.466) (end 17.937969 41.305969) (width 1) (layer B.Cu) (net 3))
 (segment (start 23.50663 21.844) (end 24.638 21.844) (width 1) (layer B.Cu) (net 3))
 (segment (start 17.937969 41.305969) (end 17.937969 26.789276) (width 1) (layer B.Cu) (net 3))
 (segment (start 17.937969 26.789276) (end 22.883245 21.844) (width 1) (layer B.Cu) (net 3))
 (segment (start 22.883245 21.844) (end 23.50663 21.844) (width 1) (layer B.Cu) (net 3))
 (via (at 29.718 45.466) (size 1.1) (drill 0.9) (layers F.Cu B.Cu) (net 3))
 (segment (start 58.928 37.084) (end 58.928 39.06951) (width 1) (layer B.Cu) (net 3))
 (segment (start 58.928 39.06951) (end 54.05551 43.942) (width 1) (layer B.Cu) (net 3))
 (via (at 40.386 43.942) (size 1.1) (drill 0.9) (layers F.Cu B.Cu) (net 3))
 (segment (start 45.89799 69.67201) (end 45.778001 69.552021) (width 1) (layer B.Cu) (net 11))
 (segment (start 45.778001 69.552021) (end 45.778001 58.361999) (width 1) (layer B.Cu) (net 11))
 (segment (start 45.778001 58.361999) (end 46.228 57.912) (width 1) (layer B.Cu) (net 11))
 (segment (start 43.053 73.706492) (end 43.053 72.517) (width 1) (layer B.Cu) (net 11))
 (segment (start 43.053 72.517) (end 45.89799 69.67201) (width 1) (layer B.Cu) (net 11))
 (segment (start 46.228 80.772) (end 46.228 76.881492) (width 1) (layer B.Cu) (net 11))
 (segment (start 46.228 76.881492) (end 43.053 73.706492) (width 1) (layer B.Cu) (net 11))
 (segment (start 53.848 80.772) (end 53.848 69.977) (width 1) (layer B.Cu) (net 12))
 (segment (start 50.038 66.167) (end 50.038 61.722) (width 1) (layer B.Cu) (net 12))
 (segment (start 53.848 69.977) (end 50.038 66.167) (width 1) (layer B.Cu) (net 12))
 (segment (start 50.038 61.722) (end 53.848 57.912) (width 1) (layer B.Cu) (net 12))
 (segment (start 61.468 80.772) (end 61.468 76.327) (width 1) (layer B.Cu) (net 13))
 (segment (start 61.468 68.072) (end 61.468 57.912) (width 1) (layer B.Cu) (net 13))
 (segment (start 61.468 76.327) (end 60.393001 75.252001) (width 1) (layer B.Cu) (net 13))
 (segment (start 60.393001 75.252001) (end 59.758001 75.252001) (width 1) (layer B.Cu) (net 13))
 (segment (start 59.758001 75.252001) (end 59.367999 74.861999) (width 1) (layer B.Cu) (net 13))
 (segment (start 59.367999 70.172001) (end 61.468 68.072) (width 1) (layer B.Cu) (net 13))
 (segment (start 59.367999 74.861999) (end 59.367999 70.172001) (width 1) (layer B.Cu) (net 13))
 (segment (start 61.468 80.772) (end 61.468 79.502) (width 0.5) (layer B.Cu) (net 13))
 (segment (start 36.322 34.036) (end 36.72802 34.44202) (width 1) (layer B.Cu) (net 14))
 (segment (start 36.72802 44.09402) (end 38.226001 45.592001) (width 1) (layer B.Cu) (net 14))
 (segment (start 36.72802 34.44202) (end 36.72802 44.09402) (width 1) (layer B.Cu) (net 14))
 (segment (start 38.226001 45.592001) (end 65.150001 45.592001) (width 1) (layer B.Cu) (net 14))
 (segment (start 65.150001 45.592001) (end 69.088 49.53) (width 1) (layer B.Cu) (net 14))
 (segment (start 69.088 49.53) (end 69.088 80.772) (width 1) (layer B.Cu) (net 14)))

